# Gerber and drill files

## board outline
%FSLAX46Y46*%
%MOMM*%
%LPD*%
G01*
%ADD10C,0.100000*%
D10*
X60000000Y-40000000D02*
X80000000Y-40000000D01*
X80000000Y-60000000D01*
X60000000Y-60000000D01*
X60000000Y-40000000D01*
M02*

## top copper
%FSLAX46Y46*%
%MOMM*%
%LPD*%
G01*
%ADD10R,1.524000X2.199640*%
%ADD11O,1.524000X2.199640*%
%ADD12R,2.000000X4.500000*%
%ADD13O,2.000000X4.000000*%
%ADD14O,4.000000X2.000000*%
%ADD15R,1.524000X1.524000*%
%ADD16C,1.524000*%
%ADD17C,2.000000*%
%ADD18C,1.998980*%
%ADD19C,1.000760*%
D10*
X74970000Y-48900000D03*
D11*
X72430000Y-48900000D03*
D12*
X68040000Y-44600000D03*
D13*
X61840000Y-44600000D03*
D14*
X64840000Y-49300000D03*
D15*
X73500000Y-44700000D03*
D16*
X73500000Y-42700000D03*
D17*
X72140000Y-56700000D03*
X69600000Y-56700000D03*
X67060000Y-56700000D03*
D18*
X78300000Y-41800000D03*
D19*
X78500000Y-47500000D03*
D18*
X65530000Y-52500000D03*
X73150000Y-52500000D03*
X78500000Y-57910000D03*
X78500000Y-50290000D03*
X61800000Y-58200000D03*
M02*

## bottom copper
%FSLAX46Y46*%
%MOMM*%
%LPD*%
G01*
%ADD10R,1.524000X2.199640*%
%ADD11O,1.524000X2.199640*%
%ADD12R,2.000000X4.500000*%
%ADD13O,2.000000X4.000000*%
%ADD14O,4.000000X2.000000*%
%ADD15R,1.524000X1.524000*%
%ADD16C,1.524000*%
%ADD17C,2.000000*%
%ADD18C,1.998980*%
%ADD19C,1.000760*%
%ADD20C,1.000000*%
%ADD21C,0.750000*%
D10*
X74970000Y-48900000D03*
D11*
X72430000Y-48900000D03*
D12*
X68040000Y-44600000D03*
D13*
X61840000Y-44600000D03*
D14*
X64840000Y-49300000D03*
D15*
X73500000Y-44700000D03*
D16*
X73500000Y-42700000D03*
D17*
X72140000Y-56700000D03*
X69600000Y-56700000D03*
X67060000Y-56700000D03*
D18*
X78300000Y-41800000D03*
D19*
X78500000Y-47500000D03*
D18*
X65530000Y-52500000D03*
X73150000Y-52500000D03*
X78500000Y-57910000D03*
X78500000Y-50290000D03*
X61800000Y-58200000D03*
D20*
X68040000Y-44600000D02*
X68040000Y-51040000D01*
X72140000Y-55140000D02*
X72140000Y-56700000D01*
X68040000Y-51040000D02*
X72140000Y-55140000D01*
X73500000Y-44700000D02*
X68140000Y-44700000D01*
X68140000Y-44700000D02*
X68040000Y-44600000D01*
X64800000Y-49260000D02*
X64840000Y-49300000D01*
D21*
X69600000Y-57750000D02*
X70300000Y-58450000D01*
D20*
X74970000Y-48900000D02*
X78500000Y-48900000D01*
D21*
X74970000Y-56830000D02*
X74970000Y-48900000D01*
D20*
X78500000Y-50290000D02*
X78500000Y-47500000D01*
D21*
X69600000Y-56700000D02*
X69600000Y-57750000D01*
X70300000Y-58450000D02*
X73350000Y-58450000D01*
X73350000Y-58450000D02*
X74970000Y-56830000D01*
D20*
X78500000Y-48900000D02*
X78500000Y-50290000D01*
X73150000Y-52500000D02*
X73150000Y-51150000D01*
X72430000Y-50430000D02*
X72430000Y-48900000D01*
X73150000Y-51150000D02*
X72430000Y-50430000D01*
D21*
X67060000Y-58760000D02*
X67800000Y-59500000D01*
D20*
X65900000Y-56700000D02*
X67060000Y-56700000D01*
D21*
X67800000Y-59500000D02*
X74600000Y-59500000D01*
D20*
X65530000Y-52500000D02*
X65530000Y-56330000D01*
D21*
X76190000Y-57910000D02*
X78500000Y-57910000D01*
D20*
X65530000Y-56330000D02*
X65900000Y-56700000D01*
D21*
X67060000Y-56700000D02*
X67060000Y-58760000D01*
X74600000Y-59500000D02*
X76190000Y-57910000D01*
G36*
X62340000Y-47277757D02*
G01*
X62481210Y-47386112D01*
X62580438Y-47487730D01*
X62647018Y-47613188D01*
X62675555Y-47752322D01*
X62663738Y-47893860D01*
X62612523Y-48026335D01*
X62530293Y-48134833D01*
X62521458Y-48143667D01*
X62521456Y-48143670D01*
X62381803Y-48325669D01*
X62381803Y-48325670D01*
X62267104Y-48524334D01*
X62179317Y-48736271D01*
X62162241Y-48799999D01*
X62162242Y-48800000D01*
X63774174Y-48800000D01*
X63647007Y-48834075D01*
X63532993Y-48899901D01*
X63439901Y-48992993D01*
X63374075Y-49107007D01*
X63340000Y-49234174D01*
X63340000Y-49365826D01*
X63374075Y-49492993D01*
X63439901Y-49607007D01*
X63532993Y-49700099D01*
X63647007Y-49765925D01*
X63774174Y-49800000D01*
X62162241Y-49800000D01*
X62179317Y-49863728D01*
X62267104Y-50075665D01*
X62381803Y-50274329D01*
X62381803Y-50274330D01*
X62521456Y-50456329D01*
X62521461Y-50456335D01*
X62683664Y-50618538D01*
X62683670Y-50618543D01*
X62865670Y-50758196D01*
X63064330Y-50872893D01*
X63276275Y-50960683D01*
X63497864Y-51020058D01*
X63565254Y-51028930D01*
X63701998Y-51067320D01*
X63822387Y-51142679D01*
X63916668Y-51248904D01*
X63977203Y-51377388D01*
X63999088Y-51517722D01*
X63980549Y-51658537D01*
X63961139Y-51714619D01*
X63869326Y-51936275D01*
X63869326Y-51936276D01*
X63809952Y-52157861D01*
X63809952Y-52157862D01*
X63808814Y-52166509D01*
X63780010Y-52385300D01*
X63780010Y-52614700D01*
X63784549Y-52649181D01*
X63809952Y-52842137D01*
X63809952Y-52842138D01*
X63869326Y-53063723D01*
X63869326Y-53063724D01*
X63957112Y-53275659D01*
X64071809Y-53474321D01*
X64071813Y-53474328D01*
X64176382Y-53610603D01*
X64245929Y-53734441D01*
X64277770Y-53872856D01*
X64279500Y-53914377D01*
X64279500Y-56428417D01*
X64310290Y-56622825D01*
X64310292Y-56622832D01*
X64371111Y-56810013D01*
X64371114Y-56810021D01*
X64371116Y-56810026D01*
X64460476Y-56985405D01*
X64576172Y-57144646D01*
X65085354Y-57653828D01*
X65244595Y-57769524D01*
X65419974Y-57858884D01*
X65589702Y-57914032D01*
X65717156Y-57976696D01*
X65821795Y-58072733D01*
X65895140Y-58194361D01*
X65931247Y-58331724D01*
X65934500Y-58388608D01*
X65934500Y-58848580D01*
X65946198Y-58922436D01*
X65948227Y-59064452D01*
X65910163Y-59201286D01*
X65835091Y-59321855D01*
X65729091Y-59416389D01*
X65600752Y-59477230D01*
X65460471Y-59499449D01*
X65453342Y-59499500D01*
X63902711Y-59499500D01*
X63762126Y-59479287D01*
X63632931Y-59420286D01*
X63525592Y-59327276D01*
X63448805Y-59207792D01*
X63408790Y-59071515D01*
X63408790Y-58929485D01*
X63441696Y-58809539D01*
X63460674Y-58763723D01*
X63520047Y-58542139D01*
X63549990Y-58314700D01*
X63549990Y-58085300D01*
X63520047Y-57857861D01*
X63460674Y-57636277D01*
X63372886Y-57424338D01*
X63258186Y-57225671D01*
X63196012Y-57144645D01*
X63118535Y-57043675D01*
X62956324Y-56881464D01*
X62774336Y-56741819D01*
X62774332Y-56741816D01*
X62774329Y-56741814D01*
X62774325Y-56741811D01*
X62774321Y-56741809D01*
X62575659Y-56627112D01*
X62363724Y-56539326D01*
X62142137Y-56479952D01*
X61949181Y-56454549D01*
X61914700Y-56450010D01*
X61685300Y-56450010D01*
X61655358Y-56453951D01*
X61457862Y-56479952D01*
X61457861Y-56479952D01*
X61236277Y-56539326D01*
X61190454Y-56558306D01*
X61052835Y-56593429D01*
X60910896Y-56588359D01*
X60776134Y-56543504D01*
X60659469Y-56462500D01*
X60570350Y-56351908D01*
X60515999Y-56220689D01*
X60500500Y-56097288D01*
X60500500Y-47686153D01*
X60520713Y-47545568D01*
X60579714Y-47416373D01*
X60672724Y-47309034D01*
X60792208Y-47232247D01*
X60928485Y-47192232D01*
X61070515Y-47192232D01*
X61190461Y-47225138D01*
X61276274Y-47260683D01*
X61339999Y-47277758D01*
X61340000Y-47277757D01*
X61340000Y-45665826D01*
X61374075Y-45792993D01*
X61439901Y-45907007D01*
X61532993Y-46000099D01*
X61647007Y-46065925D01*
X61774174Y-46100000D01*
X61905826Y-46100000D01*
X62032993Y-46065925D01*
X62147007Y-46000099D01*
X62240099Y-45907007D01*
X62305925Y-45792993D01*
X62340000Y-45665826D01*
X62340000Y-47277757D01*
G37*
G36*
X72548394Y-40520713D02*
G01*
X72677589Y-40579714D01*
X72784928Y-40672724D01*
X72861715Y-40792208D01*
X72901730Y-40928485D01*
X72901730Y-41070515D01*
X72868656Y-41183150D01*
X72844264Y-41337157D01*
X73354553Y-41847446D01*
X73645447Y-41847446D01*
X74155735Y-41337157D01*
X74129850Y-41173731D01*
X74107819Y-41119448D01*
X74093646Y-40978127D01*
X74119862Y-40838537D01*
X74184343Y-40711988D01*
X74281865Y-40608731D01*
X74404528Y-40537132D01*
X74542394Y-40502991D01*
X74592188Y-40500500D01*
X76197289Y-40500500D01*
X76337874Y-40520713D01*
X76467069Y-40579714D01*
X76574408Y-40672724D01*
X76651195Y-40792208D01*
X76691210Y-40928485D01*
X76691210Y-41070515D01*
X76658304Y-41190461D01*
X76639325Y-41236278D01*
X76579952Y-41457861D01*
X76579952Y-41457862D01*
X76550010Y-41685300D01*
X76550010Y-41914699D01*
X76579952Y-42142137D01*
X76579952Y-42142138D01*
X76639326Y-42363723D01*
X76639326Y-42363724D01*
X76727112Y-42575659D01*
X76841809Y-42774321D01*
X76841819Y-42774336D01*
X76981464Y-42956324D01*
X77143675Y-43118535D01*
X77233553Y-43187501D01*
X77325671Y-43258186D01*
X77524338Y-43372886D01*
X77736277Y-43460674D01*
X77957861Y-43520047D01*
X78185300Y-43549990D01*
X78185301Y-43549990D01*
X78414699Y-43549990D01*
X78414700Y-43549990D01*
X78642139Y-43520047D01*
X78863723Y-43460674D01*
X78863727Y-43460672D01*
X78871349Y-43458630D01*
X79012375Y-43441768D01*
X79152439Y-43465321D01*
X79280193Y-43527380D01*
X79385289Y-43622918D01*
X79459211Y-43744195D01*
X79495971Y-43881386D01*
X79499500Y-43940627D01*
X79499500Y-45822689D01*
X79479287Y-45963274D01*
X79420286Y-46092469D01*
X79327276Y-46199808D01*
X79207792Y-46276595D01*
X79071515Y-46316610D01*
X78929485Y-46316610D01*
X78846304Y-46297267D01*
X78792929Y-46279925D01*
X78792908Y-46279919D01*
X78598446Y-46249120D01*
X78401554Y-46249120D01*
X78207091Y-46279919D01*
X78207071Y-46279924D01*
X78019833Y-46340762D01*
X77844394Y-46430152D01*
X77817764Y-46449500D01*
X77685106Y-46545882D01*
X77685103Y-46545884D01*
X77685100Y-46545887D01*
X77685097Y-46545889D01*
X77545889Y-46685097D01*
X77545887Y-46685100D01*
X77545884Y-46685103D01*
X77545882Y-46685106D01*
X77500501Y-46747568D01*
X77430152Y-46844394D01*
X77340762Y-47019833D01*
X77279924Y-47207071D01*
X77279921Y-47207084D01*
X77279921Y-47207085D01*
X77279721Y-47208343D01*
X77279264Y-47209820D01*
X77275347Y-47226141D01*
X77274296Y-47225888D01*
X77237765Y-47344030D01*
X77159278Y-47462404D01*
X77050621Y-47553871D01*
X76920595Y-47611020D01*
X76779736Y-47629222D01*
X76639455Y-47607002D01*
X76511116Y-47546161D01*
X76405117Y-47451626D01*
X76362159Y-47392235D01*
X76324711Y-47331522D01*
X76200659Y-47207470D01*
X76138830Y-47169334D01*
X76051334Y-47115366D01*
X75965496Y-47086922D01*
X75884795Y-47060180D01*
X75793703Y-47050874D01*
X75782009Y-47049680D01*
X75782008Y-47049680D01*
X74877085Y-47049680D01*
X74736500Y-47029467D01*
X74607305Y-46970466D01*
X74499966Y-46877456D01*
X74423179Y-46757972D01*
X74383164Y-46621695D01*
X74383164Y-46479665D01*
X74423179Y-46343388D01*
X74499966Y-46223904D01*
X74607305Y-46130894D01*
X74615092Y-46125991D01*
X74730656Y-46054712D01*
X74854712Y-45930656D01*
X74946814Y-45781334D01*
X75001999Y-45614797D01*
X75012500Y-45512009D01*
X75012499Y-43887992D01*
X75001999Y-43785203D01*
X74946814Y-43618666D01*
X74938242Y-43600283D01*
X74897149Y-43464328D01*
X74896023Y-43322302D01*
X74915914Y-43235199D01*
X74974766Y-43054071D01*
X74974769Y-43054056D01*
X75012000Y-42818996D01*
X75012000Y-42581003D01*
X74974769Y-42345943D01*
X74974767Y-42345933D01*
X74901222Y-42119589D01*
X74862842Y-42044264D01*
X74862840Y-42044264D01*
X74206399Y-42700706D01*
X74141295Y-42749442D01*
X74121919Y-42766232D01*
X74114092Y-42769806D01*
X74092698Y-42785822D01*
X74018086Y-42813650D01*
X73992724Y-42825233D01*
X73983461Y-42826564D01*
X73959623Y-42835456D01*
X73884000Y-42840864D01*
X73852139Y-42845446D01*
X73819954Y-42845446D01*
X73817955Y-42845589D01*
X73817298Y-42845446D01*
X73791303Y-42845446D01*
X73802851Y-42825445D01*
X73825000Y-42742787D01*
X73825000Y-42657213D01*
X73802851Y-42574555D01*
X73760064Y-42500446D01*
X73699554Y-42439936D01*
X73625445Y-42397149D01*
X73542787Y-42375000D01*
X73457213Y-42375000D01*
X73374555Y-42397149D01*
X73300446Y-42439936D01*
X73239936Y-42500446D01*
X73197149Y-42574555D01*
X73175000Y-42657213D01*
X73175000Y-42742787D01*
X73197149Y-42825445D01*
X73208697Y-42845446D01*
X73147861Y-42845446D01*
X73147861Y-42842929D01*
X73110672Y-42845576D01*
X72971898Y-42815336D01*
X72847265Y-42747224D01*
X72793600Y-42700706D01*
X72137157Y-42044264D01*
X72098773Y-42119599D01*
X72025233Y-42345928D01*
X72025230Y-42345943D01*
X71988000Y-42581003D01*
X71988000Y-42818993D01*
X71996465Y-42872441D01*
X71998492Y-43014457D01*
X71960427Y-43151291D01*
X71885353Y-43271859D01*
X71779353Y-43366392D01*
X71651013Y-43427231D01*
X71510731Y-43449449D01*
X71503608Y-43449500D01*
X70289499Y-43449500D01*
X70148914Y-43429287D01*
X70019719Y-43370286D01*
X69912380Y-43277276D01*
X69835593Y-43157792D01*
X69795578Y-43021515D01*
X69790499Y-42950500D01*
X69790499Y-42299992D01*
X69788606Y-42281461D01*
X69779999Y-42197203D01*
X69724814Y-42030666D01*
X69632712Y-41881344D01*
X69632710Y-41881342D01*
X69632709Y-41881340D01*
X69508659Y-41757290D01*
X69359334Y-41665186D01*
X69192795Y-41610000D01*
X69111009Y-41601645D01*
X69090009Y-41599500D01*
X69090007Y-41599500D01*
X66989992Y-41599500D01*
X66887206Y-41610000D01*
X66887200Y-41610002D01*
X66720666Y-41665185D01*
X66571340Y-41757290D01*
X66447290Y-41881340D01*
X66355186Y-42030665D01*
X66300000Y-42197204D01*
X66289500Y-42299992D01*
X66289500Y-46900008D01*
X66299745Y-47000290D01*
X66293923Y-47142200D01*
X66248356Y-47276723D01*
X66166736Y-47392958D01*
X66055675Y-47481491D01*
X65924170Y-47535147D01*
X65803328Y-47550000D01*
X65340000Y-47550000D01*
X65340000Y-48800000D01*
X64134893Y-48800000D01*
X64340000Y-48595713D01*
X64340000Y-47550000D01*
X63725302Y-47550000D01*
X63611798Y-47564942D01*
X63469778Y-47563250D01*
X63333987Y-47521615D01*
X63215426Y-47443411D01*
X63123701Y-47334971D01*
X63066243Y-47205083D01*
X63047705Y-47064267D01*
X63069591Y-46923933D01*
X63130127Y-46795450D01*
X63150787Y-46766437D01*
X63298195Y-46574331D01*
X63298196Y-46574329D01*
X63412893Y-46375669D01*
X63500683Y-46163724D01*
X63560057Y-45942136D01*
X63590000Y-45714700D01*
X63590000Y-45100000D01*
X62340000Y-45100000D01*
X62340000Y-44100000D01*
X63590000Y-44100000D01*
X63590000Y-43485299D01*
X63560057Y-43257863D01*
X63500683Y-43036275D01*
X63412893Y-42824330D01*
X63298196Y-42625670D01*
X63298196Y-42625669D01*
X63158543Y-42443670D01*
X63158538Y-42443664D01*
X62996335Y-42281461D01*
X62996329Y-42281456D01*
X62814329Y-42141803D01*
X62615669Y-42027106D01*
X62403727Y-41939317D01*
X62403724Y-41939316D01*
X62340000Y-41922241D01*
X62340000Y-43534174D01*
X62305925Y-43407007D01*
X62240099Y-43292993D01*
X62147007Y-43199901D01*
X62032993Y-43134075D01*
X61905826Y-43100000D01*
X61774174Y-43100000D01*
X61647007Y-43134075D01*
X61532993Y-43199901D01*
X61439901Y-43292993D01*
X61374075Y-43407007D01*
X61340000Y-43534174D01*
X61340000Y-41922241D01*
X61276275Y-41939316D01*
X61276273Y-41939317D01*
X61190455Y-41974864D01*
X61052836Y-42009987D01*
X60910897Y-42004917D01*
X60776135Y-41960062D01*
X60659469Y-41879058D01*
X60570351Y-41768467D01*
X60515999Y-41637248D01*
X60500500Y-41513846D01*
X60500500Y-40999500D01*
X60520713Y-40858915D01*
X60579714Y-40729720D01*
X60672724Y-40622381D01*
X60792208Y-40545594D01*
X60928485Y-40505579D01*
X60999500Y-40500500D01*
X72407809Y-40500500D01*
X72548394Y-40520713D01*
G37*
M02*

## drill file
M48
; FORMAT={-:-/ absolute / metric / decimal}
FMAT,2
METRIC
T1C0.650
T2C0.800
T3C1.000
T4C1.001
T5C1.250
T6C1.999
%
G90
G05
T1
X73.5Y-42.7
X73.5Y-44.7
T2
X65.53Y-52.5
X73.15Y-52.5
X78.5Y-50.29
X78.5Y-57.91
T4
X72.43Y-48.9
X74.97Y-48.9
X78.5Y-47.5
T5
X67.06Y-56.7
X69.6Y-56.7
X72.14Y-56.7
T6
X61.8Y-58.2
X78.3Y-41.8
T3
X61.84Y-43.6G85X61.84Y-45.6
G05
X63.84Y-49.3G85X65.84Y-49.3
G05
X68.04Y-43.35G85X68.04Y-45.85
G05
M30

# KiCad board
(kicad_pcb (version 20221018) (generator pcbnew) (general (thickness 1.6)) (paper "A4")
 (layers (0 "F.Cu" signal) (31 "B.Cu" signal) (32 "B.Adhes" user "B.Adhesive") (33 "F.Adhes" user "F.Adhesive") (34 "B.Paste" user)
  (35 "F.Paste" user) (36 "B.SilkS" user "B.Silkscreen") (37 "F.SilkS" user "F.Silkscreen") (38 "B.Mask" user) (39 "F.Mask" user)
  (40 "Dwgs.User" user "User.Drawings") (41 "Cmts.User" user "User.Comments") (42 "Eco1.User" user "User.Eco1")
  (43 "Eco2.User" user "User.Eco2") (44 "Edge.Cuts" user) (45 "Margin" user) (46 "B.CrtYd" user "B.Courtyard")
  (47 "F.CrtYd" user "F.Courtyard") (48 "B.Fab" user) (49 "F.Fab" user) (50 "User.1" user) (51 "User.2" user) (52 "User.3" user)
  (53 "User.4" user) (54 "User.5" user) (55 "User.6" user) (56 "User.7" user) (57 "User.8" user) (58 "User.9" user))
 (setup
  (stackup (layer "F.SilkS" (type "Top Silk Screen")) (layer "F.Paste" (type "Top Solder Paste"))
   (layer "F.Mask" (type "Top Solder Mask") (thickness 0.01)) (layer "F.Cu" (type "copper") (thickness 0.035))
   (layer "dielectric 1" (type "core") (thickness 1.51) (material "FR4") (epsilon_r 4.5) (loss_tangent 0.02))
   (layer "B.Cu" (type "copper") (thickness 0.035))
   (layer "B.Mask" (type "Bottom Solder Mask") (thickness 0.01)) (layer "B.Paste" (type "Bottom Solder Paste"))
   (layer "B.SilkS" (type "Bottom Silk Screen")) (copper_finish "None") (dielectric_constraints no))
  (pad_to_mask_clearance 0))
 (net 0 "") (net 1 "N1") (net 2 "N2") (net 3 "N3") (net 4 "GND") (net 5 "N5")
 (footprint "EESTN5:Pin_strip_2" (layer "F.Cu") (at 73.7 48.9 180)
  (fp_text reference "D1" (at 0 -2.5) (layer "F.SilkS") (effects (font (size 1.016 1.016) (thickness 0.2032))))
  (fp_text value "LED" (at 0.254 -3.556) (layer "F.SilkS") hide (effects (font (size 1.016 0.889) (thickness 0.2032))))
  (pad "1" thru_hole rect (at -1.27 0 180) (size 1.524 2.19964) (drill 1.00076) (layers "*.Cu" "*.Mask" "F.SilkS") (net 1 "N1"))
  (pad "2" thru_hole oval (at 1.27 0 180) (size 1.524 2.19964) (drill 1.00076) (layers "*.Cu" "*.Mask" "F.SilkS") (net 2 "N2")))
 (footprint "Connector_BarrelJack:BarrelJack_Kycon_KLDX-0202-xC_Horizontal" (layer "F.Cu") (at 68.04 44.6)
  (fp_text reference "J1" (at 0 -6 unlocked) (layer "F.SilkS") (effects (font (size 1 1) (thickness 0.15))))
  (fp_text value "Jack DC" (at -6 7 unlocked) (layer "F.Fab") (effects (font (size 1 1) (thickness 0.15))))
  (pad "1" thru_hole rect (at 0 0) (size 2 4.5) (drill oval 1 3.5) (layers "*.Cu" "*.Mask") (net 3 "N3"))
  (pad "2" thru_hole oval (at -6.2 0) (size 2 4) (drill oval 1 3) (layers "*.Cu" "*.Mask") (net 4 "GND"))
  (pad "3" thru_hole oval (at -3.2 4.7 90) (size 2 4) (drill oval 1 3) (layers "*.Cu" "*.Mask") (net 4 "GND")))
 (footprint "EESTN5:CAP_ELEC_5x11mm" (layer "F.Cu") (at 73.5 43.7)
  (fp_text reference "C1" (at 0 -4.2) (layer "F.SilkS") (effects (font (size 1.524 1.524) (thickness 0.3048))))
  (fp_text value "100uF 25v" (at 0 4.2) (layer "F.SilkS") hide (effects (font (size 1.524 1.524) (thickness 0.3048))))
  (pad "1" thru_hole rect (at 0 1) (size 1.524 1.524) (drill 0.65) (layers "*.Cu" "*.Mask" "F.SilkS") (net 3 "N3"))
  (pad "2" thru_hole circle (at 0 -1) (size 1.524 1.524) (drill 0.65) (layers "*.Cu" "*.Mask" "F.SilkS") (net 4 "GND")))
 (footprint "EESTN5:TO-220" (layer "F.Cu") (at 69.6 56.7 180)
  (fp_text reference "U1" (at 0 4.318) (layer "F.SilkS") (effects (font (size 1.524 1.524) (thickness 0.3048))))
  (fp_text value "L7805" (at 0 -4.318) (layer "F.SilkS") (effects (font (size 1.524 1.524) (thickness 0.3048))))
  (pad "1" thru_hole circle (at -2.54 0 180) (size 2 2) (drill 1.24968) (layers "*.Cu" "*.Mask" "F.SilkS") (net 3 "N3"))
  (pad "2" thru_hole circle (at 0 0 180) (size 2 2) (drill 1.24968) (layers "*.Cu" "*.Mask" "F.SilkS") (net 1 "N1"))
  (pad "3" thru_hole circle (at 2.54 0 180) (size 2 2) (drill 1.24968) (layers "*.Cu" "*.Mask" "F.SilkS") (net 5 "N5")))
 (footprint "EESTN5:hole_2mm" (layer "F.Cu") (at 78.3 41.8)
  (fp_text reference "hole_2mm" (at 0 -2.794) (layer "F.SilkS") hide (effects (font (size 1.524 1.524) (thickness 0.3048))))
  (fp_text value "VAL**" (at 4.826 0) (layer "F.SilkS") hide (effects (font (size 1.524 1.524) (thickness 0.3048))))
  (pad "1" thru_hole circle (at 0 0) (size 1.99898 1.99898) (drill 1.99898) (layers "*.Cu" "F.SilkS")))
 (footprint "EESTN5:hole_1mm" (layer "F.Cu") (at 78.5 47.5)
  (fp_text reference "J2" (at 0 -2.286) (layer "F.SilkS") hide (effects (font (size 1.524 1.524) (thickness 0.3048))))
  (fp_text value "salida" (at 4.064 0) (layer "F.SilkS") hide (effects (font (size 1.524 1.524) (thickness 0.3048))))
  (pad "1" thru_hole circle (at 0 0) (size 1.00076 1.00076) (drill 1.00076) (layers "*.Cu" "F.SilkS") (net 1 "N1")))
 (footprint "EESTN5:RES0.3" (layer "F.Cu") (at 69.34 52.5)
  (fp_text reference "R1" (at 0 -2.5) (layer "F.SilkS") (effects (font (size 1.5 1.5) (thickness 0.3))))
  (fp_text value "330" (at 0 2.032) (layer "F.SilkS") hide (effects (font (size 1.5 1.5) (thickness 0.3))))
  (pad "1" thru_hole circle (at -3.81 0) (size 1.99898 1.99898) (drill 0.8001) (layers "*.Cu" "*.Mask" "F.SilkS") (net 5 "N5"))
  (pad "2" thru_hole circle (at 3.81 0) (size 1.99898 1.99898) (drill 0.8001) (layers "*.Cu" "*.Mask" "F.SilkS") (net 2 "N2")))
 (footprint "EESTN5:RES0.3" (layer "F.Cu") (at 78.5 54.1 90)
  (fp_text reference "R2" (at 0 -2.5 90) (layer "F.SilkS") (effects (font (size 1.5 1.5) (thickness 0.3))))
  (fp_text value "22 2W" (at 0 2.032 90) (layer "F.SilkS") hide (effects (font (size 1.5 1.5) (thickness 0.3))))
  (pad "1" thru_hole circle (at -3.81 0 90) (size 1.99898 1.99898) (drill 0.8001) (layers "*.Cu" "*.Mask" "F.SilkS") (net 5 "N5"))
  (pad "2" thru_hole circle (at 3.81 0 90) (size 1.99898 1.99898) (drill 0.8001) (layers "*.Cu" "*.Mask" "F.SilkS") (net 1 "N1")))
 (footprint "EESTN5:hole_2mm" (layer "F.Cu") (at 61.8 58.2)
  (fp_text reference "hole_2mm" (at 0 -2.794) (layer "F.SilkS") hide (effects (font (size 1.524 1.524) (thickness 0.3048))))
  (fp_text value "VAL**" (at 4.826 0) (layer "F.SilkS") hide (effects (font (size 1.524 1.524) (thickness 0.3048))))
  (pad "1" thru_hole circle (at 0 0) (size 1.99898 1.99898) (drill 1.99898) (layers "*.Cu" "F.SilkS")))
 (gr_rect (start 60 40) (end 80 60) (stroke (width 0.1) (type default)) (fill none) (layer "Edge.Cuts"))
 (segment (start 68.04 44.6) (end 68.04 51.04) (width 1) (layer "B.Cu") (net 3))
 (segment (start 72.14 55.14) (end 72.14 56.7) (width 1) (layer "B.Cu") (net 3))
 (segment (start 68.04 51.04) (end 72.14 55.14) (width 1) (layer "B.Cu") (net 3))
 (segment (start 73.5 44.7) (end 68.14 44.7) (width 1) (layer "B.Cu") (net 3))
 (segment (start 68.14 44.7) (end 68.04 44.6) (width 1) (layer "B.Cu") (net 3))
 (segment (start 64.8 49.26) (end 64.84 49.3) (width 1) (layer "B.Cu") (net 4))
 (segment (start 69.6 57.75) (end 70.3 58.45) (width 0.75) (layer "B.Cu") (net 1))
 (segment (start 74.97 48.9) (end 78.5 48.9) (width 1) (layer "B.Cu") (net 1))
 (segment (start 74.97 56.83) (end 74.97 48.9) (width 0.75) (layer "B.Cu") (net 1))
 (segment (start 78.5 50.29) (end 78.5 47.5) (width 1) (layer "B.Cu") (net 1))
 (segment (start 69.6 56.7) (end 69.6 57.75) (width 0.75) (layer "B.Cu") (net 1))
 (segment (start 70.3 58.45) (end 73.35 58.45) (width 0.75) (layer "B.Cu") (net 1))
 (segment (start 73.35 58.45) (end 74.97 56.83) (width 0.75) (layer "B.Cu") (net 1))
 (segment (start 78.5 48.9) (end 78.5 50.29) (width 1) (layer "B.Cu") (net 1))
 (segment (start 73.15 52.5) (end 73.15 51.15) (width 1) (layer "B.Cu") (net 2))
 (segment (start 72.43 50.43) (end 72.43 48.9) (width 1) (layer "B.Cu") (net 2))
 (segment (start 73.15 51.15) (end 72.43 50.43) (width 1) (layer "B.Cu") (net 2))
 (segment (start 67.06 58.76) (end 67.8 59.5) (width 0.75) (layer "B.Cu") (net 5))
 (segment (start 65.9 56.7) (end 67.06 56.7) (width 1) (layer "B.Cu") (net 5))
 (segment (start 67.8 59.5) (end 74.6 59.5) (width 0.75) (layer "B.Cu") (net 5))
 (segment (start 65.53 52.5) (end 65.53 56.33) (width 1) (layer "B.Cu") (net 5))
 (segment (start 76.19 57.91) (end 78.5 57.91) (width 0.75) (layer "B.Cu") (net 5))
 (segment (start 65.53 56.33) (end 65.9 56.7) (width 1) (layer "B.Cu") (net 5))
 (segment (start 67.06 56.7) (end 67.06 58.76) (width 0.75) (layer "B.Cu") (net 5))
 (segment (start 74.6 59.5) (end 76.19 57.91) (width 0.75) (layer "B.Cu") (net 5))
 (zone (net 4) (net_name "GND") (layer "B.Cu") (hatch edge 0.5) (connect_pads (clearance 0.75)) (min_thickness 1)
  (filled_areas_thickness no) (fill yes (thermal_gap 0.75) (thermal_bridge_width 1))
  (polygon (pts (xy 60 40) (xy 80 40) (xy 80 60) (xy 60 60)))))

